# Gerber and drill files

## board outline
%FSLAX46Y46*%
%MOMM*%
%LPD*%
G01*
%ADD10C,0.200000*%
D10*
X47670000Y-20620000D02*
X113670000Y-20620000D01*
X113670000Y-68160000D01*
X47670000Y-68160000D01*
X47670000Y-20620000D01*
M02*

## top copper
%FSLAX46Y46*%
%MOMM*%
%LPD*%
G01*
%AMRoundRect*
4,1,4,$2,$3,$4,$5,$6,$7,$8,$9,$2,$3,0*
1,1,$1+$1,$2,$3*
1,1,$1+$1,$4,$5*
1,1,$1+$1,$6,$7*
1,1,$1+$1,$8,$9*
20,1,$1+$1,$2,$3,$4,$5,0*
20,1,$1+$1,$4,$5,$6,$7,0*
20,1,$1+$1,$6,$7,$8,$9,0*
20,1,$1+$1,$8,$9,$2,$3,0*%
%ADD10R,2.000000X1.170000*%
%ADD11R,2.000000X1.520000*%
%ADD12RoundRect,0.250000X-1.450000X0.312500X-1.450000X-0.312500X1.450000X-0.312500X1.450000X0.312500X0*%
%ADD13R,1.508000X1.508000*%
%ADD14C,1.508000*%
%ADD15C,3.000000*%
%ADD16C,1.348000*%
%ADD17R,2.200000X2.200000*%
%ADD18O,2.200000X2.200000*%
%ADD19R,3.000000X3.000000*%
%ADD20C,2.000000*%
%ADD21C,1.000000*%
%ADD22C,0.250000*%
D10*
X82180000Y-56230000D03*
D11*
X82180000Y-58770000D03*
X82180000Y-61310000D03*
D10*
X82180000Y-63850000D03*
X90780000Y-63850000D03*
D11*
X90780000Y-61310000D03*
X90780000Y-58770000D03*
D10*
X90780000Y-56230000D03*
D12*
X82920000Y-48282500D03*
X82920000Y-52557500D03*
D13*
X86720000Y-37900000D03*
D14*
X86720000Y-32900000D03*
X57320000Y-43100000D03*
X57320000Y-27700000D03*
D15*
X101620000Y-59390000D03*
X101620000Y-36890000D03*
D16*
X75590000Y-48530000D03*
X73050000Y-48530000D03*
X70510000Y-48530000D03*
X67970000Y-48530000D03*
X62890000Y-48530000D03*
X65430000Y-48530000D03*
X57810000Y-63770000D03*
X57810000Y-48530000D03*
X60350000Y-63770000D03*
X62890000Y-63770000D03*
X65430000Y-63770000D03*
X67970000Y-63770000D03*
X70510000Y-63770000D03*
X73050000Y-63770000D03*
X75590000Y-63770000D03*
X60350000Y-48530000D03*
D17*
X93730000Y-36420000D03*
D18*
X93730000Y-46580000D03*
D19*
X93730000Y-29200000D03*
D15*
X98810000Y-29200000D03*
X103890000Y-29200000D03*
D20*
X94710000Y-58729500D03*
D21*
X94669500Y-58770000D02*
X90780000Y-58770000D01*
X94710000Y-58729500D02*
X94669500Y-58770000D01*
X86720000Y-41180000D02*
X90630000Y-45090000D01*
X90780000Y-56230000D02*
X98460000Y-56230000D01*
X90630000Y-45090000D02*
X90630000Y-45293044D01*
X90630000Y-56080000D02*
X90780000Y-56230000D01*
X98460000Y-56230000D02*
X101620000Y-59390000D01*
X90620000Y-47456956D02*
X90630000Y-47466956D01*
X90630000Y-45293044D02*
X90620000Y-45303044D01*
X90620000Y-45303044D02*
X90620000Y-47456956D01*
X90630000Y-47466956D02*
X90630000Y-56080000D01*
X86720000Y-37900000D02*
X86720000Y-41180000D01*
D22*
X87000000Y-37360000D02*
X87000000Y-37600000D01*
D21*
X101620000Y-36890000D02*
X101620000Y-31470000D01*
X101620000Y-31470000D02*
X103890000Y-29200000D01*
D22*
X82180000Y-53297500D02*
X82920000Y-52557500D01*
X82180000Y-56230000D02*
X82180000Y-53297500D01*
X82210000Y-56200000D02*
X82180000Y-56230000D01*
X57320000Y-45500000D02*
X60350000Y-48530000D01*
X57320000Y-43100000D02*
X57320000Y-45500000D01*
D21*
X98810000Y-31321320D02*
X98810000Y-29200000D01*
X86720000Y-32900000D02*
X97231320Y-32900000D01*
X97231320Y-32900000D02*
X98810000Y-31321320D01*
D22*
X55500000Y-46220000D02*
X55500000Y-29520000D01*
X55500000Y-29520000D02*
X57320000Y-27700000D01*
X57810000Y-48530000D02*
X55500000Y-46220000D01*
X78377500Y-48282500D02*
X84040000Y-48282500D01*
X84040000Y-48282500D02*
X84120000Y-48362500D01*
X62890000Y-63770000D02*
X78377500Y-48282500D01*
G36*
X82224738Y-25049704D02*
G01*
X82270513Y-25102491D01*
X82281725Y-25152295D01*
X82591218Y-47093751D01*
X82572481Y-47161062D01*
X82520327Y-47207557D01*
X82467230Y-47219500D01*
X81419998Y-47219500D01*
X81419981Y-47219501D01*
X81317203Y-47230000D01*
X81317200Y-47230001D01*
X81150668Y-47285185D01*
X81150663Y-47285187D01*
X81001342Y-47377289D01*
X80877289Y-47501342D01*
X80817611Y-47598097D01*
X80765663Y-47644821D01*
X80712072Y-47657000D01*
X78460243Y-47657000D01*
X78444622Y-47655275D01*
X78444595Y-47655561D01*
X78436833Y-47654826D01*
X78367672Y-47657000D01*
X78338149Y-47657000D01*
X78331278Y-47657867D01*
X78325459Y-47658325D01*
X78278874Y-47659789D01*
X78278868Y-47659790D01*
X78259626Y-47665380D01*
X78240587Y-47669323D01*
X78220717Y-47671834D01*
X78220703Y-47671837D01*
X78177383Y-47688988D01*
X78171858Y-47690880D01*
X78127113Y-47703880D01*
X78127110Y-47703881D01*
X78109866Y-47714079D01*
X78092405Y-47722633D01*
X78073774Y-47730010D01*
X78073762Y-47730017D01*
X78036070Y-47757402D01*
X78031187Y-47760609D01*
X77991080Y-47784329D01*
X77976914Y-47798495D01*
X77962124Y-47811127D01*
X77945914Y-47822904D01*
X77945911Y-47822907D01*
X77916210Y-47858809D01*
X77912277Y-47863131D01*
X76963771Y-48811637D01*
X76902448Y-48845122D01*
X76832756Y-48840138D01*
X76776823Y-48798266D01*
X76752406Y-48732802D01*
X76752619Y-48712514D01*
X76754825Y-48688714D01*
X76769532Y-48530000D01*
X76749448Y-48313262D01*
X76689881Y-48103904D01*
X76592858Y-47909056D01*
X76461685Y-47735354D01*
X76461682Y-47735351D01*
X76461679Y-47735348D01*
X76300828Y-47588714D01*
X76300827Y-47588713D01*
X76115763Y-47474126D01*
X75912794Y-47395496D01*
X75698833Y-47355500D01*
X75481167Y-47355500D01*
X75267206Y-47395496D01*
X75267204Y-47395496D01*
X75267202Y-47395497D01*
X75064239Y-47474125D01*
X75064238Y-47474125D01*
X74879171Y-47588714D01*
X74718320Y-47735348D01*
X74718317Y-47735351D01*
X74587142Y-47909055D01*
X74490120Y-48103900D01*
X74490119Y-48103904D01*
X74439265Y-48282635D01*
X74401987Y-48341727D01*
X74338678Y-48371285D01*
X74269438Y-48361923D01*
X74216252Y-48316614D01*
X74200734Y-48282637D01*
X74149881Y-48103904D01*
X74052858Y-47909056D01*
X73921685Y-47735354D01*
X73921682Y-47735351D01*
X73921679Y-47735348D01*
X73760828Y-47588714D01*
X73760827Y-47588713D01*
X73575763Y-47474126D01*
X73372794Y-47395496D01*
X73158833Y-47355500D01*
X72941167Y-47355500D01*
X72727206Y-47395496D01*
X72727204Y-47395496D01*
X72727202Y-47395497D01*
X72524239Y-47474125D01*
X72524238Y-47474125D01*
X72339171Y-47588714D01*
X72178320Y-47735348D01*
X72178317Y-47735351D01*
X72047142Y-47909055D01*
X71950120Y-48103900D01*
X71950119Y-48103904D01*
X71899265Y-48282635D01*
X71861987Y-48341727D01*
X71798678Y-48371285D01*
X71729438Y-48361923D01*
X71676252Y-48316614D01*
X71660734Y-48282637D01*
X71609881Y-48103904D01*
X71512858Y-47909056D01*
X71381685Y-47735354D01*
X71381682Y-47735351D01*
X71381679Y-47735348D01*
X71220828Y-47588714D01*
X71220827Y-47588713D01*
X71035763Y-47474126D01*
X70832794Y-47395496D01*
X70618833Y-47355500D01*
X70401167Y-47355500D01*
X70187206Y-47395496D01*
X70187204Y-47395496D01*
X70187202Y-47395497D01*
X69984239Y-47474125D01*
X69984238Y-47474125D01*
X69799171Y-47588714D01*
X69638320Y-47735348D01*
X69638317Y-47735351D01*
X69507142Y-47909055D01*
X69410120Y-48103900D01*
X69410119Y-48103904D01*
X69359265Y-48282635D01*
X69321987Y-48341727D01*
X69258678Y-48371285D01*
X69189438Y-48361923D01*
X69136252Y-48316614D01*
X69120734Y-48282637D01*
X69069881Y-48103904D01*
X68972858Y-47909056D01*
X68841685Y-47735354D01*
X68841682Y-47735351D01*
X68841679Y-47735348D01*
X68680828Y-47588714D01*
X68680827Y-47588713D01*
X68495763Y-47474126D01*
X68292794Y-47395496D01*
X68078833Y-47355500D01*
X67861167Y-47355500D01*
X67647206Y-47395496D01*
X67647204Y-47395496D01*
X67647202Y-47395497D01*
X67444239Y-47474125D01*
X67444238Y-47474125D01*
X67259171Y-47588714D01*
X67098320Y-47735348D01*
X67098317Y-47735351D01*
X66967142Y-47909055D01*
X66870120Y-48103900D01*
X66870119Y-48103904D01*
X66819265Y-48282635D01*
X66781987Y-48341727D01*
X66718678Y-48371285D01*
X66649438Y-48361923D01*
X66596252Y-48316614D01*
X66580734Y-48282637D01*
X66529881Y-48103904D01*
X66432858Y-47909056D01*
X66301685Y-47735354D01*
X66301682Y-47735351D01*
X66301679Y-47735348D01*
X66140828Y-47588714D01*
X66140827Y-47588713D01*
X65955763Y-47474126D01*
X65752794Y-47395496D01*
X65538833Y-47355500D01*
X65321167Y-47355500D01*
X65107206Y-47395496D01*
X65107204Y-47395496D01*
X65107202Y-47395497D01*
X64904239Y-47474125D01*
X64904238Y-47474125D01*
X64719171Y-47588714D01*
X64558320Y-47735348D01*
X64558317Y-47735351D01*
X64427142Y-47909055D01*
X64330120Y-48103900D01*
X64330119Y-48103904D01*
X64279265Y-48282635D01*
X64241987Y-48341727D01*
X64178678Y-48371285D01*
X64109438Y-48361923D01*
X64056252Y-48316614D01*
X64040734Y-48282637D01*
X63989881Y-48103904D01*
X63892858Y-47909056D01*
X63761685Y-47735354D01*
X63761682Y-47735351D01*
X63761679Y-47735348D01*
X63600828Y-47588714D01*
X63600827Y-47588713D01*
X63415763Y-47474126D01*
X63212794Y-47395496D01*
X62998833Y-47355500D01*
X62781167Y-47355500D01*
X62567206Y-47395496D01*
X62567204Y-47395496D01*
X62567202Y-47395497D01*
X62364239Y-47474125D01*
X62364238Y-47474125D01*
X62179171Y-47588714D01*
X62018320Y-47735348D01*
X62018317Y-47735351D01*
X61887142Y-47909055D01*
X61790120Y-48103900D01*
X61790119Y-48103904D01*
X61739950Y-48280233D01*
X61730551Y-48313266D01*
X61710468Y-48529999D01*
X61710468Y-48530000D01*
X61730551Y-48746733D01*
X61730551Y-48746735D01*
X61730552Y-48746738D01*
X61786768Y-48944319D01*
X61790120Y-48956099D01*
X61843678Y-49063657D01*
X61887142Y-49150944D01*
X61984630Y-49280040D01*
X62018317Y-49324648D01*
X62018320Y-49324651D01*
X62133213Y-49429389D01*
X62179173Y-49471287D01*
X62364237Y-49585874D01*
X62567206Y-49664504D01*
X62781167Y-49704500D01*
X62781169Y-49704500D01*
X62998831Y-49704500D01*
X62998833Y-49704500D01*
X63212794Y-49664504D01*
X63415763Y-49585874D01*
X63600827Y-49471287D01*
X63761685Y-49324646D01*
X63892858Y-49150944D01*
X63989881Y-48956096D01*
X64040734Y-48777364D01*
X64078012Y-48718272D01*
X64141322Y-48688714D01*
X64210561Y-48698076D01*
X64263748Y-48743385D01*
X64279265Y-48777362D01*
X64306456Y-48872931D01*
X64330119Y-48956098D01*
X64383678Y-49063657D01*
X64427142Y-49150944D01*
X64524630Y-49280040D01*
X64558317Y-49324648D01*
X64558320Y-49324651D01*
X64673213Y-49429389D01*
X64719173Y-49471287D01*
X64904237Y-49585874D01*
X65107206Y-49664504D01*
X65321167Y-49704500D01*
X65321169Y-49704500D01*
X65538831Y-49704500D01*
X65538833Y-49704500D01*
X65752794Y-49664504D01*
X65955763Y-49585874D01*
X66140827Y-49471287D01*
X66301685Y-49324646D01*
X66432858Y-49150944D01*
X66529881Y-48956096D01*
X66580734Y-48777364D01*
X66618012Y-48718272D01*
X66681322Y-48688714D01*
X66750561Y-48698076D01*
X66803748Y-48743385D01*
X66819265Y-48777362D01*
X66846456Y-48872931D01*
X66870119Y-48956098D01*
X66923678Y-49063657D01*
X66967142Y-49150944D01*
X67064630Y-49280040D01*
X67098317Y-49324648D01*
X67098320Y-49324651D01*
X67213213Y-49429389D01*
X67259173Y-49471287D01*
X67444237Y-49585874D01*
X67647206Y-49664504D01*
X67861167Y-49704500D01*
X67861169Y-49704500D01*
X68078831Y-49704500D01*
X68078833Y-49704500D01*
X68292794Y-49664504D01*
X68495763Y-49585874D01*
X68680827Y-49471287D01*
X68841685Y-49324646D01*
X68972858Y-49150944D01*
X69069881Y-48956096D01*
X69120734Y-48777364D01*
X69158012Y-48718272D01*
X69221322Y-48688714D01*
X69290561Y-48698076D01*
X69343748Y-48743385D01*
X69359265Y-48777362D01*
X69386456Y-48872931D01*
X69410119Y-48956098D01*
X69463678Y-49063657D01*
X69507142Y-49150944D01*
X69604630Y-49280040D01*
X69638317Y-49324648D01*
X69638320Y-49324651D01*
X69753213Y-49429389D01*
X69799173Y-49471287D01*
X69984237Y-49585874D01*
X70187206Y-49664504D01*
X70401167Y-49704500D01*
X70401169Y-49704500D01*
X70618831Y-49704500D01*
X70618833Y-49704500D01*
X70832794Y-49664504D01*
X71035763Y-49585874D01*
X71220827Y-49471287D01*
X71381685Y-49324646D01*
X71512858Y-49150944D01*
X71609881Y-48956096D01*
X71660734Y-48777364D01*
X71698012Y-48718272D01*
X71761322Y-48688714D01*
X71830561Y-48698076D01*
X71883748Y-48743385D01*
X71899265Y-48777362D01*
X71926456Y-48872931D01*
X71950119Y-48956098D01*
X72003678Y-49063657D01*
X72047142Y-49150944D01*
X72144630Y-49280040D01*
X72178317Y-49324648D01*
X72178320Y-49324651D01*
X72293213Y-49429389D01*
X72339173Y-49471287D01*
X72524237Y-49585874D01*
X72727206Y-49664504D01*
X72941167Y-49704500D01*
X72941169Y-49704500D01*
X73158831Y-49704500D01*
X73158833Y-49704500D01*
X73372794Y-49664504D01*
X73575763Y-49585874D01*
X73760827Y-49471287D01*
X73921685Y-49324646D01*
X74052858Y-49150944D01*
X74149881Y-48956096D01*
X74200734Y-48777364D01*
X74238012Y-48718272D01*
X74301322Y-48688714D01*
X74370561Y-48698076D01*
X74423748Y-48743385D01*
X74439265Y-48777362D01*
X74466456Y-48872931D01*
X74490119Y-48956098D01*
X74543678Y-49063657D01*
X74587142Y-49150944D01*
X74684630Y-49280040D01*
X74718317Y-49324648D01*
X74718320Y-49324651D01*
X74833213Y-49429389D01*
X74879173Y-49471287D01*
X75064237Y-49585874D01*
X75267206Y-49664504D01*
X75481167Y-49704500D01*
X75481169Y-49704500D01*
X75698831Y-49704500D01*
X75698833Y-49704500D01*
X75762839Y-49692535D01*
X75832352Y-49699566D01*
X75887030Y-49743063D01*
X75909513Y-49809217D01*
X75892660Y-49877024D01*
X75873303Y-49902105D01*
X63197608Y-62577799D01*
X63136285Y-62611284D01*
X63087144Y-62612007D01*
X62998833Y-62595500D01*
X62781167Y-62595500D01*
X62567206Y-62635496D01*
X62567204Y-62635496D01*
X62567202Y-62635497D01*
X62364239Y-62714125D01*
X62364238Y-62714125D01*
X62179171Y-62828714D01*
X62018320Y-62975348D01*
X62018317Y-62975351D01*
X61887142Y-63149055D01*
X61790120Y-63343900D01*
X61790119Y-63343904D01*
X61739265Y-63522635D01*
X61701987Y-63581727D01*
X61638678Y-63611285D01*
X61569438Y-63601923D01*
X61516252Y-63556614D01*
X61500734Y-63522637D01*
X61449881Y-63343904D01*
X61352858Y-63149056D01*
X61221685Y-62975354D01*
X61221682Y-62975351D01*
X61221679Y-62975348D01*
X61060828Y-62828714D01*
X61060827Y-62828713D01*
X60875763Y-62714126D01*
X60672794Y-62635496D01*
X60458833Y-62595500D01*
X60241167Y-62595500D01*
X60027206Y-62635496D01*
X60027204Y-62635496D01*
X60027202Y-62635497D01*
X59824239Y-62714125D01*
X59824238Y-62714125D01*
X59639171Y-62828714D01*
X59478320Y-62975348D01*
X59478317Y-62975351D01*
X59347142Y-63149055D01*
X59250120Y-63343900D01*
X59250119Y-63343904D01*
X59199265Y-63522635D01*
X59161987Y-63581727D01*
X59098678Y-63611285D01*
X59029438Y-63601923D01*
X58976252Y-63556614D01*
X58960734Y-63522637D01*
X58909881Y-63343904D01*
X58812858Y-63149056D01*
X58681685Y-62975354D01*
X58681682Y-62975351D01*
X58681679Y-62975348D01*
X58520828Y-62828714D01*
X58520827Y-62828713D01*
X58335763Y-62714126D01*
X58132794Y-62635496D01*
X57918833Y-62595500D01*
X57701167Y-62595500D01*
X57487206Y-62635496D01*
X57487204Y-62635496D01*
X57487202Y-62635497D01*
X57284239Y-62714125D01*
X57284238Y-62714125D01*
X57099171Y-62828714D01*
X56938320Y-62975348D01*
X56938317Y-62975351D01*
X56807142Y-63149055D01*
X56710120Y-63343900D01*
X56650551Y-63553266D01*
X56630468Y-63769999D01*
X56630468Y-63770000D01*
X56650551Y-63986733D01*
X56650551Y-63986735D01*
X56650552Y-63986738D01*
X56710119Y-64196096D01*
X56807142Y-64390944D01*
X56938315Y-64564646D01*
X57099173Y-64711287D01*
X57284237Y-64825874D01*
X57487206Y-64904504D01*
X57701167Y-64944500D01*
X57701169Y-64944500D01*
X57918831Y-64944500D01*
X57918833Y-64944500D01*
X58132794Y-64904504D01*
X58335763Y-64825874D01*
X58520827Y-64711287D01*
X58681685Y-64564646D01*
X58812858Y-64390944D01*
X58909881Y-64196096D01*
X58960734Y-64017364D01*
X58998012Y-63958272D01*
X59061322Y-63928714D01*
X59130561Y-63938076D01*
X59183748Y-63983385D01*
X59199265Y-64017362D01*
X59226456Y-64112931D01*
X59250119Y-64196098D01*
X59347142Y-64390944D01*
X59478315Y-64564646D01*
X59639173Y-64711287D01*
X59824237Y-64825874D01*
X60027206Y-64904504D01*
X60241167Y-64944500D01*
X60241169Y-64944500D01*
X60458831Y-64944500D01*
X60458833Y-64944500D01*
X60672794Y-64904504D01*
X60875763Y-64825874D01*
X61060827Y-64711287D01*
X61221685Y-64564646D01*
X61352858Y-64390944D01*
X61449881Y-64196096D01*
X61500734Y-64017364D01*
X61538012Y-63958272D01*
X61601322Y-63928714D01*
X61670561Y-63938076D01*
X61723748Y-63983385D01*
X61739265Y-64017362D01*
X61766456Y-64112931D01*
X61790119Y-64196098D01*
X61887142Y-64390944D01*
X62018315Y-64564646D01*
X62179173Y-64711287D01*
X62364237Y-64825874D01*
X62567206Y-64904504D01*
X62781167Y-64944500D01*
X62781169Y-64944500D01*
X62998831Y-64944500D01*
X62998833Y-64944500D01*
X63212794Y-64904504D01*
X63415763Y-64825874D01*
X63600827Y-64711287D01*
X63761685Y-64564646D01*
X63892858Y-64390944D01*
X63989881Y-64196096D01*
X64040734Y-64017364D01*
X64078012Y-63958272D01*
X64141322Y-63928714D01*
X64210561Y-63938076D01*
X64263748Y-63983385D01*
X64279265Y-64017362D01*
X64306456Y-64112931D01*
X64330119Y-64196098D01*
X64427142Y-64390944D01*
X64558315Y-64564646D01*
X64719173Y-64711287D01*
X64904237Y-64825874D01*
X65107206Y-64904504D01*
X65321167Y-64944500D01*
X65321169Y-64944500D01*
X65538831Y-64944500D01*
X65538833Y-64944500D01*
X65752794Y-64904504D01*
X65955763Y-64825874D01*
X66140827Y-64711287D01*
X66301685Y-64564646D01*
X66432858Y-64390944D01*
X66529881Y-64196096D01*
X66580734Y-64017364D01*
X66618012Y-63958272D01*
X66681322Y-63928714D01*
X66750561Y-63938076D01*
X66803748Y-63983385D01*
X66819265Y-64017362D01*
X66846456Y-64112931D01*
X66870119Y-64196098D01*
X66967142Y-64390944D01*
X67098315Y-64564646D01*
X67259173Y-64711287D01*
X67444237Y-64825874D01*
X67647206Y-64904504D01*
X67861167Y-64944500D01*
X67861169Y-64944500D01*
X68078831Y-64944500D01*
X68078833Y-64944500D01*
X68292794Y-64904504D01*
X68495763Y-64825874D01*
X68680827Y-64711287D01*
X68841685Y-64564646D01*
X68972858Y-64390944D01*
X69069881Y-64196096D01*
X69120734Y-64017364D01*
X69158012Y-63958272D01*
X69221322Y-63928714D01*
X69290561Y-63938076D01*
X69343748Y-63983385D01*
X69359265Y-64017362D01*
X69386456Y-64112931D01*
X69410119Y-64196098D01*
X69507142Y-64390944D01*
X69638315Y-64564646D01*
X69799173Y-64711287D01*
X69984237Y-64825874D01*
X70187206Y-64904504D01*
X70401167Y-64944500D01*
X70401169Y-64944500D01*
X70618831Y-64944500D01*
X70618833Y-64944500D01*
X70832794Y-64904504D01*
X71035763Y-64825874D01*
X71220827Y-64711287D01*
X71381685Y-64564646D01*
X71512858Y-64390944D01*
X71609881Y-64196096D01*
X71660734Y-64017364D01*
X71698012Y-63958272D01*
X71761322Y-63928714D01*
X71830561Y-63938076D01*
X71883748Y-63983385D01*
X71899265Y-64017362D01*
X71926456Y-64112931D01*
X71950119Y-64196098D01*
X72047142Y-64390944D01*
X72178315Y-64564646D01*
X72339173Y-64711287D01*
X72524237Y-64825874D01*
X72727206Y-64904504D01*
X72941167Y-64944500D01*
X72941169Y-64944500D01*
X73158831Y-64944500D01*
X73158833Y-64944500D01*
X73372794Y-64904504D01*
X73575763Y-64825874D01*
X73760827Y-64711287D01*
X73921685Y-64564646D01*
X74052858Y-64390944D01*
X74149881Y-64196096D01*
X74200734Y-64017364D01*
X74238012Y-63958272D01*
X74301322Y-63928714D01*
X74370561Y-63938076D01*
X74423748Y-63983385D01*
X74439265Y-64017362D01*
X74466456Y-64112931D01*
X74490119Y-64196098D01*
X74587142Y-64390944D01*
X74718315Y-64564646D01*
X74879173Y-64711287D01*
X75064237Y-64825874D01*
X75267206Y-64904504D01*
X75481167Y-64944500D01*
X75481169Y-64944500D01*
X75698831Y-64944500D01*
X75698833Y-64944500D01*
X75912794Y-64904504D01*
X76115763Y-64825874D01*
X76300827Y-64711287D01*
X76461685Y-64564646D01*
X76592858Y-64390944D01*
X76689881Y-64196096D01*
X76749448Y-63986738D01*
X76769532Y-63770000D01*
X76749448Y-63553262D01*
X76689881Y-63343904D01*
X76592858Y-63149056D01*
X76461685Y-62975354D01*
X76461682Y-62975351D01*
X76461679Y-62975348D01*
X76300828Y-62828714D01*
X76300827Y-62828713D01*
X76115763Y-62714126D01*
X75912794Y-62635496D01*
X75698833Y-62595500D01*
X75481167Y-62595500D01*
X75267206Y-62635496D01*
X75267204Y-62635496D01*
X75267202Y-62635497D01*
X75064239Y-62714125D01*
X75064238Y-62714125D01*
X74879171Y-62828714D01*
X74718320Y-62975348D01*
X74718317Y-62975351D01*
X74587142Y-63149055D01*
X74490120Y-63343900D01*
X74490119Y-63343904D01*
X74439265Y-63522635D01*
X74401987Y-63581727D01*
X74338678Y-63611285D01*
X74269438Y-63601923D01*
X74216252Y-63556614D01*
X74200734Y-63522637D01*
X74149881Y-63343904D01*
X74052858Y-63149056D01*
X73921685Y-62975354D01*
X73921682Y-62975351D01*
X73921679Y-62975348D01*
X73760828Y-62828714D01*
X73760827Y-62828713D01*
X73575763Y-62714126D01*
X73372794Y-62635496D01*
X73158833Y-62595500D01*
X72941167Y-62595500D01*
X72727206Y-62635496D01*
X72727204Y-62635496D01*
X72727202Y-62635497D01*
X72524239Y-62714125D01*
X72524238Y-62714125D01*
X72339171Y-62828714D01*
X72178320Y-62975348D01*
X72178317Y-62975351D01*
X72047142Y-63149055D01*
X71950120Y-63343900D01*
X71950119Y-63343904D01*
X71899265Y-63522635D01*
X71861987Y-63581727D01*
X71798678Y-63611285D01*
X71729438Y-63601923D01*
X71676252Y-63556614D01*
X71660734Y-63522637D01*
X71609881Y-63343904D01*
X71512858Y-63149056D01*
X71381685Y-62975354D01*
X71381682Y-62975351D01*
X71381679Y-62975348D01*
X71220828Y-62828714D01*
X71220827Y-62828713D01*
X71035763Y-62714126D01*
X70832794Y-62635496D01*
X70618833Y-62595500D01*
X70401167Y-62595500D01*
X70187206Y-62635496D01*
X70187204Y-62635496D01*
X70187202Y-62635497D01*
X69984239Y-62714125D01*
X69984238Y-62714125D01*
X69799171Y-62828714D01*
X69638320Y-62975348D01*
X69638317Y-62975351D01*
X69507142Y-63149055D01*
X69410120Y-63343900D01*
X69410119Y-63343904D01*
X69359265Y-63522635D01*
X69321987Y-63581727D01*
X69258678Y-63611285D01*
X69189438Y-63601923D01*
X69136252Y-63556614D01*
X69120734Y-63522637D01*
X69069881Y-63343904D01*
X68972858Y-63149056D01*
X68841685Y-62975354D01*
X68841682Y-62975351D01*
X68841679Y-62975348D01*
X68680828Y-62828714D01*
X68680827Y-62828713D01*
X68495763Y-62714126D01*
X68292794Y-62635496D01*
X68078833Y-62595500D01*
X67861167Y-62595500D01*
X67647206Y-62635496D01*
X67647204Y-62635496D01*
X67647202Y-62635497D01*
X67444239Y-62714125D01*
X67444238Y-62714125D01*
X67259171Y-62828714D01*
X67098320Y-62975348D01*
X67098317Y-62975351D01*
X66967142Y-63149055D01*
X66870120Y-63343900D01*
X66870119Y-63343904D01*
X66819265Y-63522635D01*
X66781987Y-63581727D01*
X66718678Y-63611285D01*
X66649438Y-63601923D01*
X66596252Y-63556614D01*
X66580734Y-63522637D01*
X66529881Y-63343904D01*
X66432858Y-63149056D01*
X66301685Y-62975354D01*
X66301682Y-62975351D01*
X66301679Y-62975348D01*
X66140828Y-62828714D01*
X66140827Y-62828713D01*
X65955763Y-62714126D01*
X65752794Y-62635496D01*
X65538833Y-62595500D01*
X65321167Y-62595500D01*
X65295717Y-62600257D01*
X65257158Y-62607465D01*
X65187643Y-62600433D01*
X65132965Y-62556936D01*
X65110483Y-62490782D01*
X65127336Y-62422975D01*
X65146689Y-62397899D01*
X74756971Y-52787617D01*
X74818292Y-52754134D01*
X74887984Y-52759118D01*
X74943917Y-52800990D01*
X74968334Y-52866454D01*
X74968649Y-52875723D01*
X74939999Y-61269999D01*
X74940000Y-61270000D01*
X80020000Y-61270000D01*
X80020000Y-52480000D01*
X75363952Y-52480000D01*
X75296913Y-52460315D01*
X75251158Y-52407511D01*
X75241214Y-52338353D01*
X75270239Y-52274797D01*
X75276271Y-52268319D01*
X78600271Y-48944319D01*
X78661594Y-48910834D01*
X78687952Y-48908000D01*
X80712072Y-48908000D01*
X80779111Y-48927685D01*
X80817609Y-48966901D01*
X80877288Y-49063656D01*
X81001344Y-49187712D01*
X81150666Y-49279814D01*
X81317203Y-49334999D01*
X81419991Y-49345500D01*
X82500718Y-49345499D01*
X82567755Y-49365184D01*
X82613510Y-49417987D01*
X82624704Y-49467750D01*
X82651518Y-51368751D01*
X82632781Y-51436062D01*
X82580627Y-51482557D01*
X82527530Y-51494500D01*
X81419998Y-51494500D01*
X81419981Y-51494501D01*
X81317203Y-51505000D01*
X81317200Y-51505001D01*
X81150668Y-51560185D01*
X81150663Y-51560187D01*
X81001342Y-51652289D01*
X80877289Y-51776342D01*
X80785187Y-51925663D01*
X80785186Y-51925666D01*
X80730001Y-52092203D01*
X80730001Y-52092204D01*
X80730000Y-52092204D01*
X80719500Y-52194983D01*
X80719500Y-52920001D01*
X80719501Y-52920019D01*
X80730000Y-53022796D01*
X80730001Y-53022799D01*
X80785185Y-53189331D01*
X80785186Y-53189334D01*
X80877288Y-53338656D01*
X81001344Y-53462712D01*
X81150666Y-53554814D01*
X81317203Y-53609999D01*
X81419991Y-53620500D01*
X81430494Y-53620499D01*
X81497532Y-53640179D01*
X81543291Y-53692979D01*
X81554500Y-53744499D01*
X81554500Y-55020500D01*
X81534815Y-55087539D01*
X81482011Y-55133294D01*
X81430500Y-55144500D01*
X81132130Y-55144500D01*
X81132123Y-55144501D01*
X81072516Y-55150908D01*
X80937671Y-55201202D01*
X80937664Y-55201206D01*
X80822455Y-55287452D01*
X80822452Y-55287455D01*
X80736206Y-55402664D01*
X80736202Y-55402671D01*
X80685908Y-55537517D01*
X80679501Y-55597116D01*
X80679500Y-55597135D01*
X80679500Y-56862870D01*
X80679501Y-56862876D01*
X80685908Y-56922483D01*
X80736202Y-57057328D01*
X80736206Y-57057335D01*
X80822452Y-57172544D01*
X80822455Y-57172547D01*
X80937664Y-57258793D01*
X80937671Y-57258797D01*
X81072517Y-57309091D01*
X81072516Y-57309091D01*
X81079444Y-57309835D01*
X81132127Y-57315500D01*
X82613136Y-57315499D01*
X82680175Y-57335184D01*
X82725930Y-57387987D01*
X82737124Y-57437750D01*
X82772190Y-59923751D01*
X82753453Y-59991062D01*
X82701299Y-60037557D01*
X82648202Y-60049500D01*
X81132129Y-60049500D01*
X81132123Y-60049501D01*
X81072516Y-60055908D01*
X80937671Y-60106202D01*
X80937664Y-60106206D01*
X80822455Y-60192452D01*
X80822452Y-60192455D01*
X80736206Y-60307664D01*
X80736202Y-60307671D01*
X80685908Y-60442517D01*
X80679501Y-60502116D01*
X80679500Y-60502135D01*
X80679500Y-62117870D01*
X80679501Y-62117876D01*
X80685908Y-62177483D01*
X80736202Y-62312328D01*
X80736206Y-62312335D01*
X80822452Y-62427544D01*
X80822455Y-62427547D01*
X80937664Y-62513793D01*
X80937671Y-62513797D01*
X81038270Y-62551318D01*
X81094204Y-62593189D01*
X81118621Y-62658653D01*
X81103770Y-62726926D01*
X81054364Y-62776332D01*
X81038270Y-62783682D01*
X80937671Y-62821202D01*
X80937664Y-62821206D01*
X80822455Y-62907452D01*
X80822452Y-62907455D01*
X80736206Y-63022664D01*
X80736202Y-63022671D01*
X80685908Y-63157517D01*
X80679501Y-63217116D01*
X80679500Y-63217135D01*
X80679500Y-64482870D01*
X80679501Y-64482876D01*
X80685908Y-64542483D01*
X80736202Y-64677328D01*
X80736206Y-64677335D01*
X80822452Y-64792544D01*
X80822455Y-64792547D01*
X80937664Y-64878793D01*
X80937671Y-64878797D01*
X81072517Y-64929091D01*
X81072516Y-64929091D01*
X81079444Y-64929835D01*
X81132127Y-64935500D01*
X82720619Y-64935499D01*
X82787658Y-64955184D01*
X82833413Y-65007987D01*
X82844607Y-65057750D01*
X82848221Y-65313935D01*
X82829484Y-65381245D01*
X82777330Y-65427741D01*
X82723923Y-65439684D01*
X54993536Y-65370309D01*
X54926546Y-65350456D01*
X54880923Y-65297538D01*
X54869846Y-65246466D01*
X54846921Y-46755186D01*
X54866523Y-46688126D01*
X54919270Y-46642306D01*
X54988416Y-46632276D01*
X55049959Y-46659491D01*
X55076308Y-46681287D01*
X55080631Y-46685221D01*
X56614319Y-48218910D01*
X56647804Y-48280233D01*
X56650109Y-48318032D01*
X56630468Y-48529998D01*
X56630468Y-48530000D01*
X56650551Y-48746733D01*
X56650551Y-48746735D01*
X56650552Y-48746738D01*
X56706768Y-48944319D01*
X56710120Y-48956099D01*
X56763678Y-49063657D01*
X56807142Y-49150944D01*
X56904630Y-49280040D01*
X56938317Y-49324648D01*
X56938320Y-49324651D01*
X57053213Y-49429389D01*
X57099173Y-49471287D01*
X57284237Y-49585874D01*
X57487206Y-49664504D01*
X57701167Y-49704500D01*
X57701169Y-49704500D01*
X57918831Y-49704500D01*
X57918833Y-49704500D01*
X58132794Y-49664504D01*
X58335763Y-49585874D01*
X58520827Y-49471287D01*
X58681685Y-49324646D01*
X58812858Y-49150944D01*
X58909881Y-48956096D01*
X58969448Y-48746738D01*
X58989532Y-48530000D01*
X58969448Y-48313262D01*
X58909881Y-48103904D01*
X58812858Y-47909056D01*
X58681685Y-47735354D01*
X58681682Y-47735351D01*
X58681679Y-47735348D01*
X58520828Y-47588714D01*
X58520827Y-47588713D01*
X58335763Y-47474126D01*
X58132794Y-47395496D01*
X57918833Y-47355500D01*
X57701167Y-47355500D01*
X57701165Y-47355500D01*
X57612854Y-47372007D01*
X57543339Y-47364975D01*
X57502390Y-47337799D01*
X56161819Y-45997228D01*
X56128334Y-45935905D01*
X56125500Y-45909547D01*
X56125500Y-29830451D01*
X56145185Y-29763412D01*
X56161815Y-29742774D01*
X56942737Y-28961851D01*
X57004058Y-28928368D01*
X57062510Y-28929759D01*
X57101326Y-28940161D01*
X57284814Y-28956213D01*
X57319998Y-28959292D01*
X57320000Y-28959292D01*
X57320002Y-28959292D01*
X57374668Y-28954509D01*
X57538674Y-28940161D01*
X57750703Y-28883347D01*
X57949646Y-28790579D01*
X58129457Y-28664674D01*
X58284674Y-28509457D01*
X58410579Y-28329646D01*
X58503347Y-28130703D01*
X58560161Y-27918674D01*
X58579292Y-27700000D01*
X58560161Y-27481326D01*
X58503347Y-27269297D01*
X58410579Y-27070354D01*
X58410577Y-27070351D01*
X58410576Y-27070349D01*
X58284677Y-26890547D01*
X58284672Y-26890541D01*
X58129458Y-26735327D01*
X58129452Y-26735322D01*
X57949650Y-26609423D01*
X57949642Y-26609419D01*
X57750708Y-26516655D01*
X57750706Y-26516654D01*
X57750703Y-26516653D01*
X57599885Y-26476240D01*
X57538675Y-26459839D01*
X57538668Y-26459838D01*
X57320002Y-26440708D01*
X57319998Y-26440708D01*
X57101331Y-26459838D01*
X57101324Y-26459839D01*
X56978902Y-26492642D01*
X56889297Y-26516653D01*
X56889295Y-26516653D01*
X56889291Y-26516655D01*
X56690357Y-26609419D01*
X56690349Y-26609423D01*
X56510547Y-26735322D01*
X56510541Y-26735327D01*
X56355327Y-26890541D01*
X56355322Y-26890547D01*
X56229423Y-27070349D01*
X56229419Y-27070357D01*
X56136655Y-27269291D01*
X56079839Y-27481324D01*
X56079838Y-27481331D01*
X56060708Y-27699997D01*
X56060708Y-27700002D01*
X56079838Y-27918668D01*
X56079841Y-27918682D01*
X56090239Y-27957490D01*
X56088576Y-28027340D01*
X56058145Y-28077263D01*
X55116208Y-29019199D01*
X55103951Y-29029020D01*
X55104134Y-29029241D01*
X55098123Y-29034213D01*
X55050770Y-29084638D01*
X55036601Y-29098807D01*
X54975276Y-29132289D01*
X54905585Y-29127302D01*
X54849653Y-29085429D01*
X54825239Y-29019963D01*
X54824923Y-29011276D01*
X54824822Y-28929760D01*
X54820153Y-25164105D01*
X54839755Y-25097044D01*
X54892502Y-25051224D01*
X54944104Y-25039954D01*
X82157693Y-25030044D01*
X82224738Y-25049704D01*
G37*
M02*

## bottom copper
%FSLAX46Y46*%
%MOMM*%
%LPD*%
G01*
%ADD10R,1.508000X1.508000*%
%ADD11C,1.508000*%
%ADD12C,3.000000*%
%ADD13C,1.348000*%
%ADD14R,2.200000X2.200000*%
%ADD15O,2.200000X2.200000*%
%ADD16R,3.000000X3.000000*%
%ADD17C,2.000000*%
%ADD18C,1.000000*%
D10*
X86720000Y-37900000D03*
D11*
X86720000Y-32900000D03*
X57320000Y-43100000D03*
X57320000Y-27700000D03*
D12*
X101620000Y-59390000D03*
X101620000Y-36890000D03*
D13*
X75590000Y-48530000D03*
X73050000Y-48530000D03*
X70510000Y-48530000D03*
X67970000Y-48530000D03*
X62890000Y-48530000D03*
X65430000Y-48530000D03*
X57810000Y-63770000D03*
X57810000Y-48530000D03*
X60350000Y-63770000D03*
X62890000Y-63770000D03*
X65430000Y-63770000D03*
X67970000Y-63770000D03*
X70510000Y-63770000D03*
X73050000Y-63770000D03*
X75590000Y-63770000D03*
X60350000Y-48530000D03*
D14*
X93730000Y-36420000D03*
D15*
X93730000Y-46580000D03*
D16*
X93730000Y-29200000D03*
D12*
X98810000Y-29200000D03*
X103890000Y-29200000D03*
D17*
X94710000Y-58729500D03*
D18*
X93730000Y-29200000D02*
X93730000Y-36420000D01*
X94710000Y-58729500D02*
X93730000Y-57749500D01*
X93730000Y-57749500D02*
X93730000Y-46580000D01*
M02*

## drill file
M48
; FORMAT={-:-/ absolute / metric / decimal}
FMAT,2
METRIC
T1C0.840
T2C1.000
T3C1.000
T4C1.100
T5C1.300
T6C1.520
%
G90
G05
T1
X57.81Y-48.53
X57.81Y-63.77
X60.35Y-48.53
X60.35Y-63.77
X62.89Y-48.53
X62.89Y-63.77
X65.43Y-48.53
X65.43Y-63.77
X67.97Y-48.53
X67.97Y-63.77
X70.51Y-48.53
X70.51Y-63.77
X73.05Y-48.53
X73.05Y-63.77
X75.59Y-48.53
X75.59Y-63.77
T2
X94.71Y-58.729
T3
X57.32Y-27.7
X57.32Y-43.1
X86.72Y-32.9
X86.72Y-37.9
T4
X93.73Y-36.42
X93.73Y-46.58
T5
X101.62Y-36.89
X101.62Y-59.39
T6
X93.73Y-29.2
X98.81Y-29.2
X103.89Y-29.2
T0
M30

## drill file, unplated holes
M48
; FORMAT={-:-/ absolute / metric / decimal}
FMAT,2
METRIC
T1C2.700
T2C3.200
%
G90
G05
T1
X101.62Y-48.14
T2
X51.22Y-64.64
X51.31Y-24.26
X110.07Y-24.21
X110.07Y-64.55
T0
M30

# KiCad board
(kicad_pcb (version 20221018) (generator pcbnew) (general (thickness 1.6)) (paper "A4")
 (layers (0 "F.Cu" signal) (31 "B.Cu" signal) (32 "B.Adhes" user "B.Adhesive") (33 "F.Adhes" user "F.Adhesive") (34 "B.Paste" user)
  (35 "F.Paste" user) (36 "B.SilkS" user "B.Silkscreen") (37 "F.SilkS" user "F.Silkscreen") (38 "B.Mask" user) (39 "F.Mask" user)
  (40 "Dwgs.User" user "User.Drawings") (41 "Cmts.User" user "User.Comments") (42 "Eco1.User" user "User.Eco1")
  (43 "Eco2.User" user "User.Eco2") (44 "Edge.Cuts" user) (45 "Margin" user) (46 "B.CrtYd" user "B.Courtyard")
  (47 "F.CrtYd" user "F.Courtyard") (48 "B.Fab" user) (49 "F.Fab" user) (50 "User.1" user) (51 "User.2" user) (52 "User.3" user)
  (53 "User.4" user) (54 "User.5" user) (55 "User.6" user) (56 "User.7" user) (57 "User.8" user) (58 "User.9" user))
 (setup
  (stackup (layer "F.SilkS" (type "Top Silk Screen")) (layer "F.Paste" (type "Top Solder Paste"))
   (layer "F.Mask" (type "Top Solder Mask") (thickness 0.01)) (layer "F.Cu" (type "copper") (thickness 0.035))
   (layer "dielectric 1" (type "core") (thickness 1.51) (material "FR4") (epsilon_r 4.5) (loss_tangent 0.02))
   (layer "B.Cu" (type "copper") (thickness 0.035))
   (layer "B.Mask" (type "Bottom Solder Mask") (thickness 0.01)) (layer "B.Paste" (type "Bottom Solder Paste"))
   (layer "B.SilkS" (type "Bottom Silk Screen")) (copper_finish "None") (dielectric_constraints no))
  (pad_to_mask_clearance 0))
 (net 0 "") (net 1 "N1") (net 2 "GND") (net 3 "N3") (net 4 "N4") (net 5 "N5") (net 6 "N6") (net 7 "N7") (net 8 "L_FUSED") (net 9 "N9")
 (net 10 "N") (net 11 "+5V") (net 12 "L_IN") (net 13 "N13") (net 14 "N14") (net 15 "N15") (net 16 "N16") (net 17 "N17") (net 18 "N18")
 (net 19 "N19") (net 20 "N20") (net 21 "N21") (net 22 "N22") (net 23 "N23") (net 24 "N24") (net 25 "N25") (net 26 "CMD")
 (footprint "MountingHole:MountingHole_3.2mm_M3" (layer "F.Cu") (at 110.07 24.21)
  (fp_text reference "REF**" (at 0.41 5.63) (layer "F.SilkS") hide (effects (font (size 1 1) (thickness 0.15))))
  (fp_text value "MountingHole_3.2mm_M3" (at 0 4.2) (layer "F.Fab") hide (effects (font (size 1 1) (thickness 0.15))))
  (pad "" np_thru_hole circle (at 0 0) (size 3.2 3.2) (drill 3.2) (layers "F&B.Cu" "*.Mask")))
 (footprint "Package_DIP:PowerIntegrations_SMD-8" (layer "F.Cu") (at 86.48 60.04)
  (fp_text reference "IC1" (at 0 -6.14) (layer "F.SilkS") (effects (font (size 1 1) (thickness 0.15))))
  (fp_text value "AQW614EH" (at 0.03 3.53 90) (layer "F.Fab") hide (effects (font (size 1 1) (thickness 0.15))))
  (pad "1" smd rect (at -4.3 -3.81) (size 2 1.17) (layers "F.Cu" "F.Paste" "F.Mask") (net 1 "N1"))
  (pad "2" smd rect (at -4.3 -1.27) (size 2 1.52) (layers "F.Cu" "F.Paste" "F.Mask") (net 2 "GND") (zone_connect 2))
  (pad "3" smd rect (at -4.3 1.27) (size 2 1.52) (layers "F.Cu" "F.Paste" "F.Mask") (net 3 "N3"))
  (pad "4" smd rect (at -4.3 3.81) (size 2 1.17) (layers "F.Cu" "F.Paste" "F.Mask") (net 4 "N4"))
  (pad "5" smd rect (at 4.3 3.81) (size 2 1.17) (layers "F.Cu" "F.Paste" "F.Mask") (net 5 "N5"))
  (pad "6" smd rect (at 4.3 1.27) (size 2 1.52) (layers "F.Cu" "F.Paste" "F.Mask") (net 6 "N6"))
  (pad "7" smd rect (at 4.3 -1.27) (size 2 1.52) (layers "F.Cu" "F.Paste" "F.Mask") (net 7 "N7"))
  (pad "8" smd rect (at 4.3 -3.81) (size 2 1.17) (layers "F.Cu" "F.Paste" "F.Mask") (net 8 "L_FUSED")))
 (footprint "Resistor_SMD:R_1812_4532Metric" (layer "F.Cu") (at 82.92 50.42 -90)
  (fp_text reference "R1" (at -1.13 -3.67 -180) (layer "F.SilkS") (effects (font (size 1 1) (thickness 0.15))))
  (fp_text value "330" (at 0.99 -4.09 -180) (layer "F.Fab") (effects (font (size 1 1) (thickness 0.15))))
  (pad "1" smd roundrect (at -2.1375 0 270) (size 1.125 3.4) (layers "F.Cu" "F.Paste" "F.Mask") (roundrect_rratio 0.2222222222) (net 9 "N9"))
  (pad "2" smd roundrect (at 2.1375 0 270) (size 1.125 3.4) (layers "F.Cu" "F.Paste" "F.Mask") (roundrect_rratio 0.2222222222) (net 1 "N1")))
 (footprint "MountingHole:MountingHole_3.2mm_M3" (layer "F.Cu") (at 110.07 64.55)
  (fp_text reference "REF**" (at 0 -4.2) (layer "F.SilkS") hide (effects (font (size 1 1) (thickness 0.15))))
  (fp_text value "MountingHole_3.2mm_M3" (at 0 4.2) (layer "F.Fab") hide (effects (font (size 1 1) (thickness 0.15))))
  (pad "" np_thru_hole circle (at 0 0) (size 3.2 3.2) (drill 3.2) (layers "F&B.Cu" "*.Mask")))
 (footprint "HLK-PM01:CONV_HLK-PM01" (layer "F.Cu") (at 72.02 35.4 180)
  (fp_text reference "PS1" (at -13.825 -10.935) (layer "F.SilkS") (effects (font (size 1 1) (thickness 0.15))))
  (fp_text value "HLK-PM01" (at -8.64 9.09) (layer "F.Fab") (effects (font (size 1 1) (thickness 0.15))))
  (pad "1" thru_hole rect (at -14.7 -2.5 180) (size 1.508 1.508) (drill 1) (layers "*.Cu" "*.Mask") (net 8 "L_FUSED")
   (solder_mask_margin 0.102))
  (pad "2" thru_hole circle (at -14.7 2.5 180) (size 1.508 1.508) (drill 1) (layers "*.Cu" "*.Mask") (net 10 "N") (solder_mask_margin 0.102))
  (pad "3" thru_hole circle (at 14.7 -7.7 180) (size 1.508 1.508) (drill 1) (layers "*.Cu" "*.Mask") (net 2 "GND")
   (solder_mask_margin 0.102) (zone_connect 2))
  (pad "4" thru_hole circle (at 14.7 7.7 180) (size 1.508 1.508) (drill 1) (layers "*.Cu" "*.Mask") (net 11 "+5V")
   (solder_mask_margin 0.102)))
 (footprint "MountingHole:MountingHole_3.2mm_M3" (layer "F.Cu") (at 51.22 64.64)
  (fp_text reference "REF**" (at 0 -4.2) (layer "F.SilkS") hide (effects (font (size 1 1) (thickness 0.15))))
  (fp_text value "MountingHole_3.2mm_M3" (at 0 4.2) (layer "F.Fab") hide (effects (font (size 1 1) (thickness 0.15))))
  (pad "" np_thru_hole circle (at 0 0) (size 3.2 3.2) (drill 3.2) (layers "F&B.Cu" "*.Mask")))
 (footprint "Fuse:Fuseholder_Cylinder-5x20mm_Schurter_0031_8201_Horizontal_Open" (layer "F.Cu") (at 101.62 59.39 90)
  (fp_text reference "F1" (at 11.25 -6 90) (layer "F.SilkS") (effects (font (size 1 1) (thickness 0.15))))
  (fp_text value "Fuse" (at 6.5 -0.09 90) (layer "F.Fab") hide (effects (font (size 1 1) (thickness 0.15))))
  (pad "" np_thru_hole circle (at 11.25 0 90) (size 2.7 2.7) (drill 2.7) (layers "*.Cu" "*.Mask"))
  (pad "1" thru_hole circle (at 0 0 90) (size 3 3) (drill 1.3) (layers "*.Cu" "*.Mask") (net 8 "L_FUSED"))
  (pad "2" thru_hole circle (at 22.5 0 90) (size 3 3) (drill 1.3) (layers "*.Cu" "*.Mask") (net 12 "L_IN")))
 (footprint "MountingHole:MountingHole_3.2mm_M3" (layer "F.Cu") (at 51.31 24.26)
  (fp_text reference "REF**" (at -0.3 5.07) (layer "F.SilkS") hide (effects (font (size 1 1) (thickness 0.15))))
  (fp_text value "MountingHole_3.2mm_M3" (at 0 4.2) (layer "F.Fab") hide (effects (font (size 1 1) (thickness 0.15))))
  (pad "" np_thru_hole circle (at 0 0) (size 3.2 3.2) (drill 3.2) (layers "*.Cu" "*.Mask")))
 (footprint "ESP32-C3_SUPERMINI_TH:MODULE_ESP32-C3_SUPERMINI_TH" (layer "F.Cu") (at 67.71 56.15 90)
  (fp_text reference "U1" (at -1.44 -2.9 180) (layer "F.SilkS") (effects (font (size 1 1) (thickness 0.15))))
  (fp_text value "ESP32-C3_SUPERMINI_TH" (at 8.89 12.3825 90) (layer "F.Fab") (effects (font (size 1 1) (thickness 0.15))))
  (pad "0" thru_hole circle (at 7.62 7.88 90) (size 1.348 1.348) (drill 0.84) (layers "*.Cu" "*.Mask") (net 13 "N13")
   (solder_mask_margin 0.102))
  (pad "1" thru_hole circle (at 7.62 5.34 90) (size 1.348 1.348) (drill 0.84) (layers "*.Cu" "*.Mask") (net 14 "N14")
   (solder_mask_margin 0.102))
  (pad "2" thru_hole circle (at 7.62 2.8 90) (size 1.348 1.348) (drill 0.84) (layers "*.Cu" "*.Mask") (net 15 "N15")
   (solder_mask_margin 0.102))
  (pad "3" thru_hole circle (at 7.62 0.26 90) (size 1.348 1.348) (drill 0.84) (layers "*.Cu" "*.Mask") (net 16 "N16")
   (solder_mask_margin 0.102))
  (pad "3.3" thru_hole circle (at 7.62 -4.82 90) (size 1.348 1.348) (drill 0.84) (layers "*.Cu" "*.Mask") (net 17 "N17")
   (solder_mask_margin 0.102))
  (pad "4" thru_hole circle (at 7.62 -2.28 90) (size 1.348 1.348) (drill 0.84) (layers "*.Cu" "*.Mask") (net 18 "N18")
   (solder_mask_margin 0.102))
  (pad "5" thru_hole circle (at -7.62 -9.9 90) (size 1.348 1.348) (drill 0.84) (layers "*.Cu" "*.Mask") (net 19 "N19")
   (solder_mask_margin 0.102))
  (pad "5V" thru_hole circle (at 7.62 -9.9 90) (size 1.348 1.348) (drill 0.84) (layers "*.Cu" "*.Mask") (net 11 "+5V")
   (solder_mask_margin 0.102))
  (pad "6" thru_hole circle (at -7.62 -7.36 90) (size 1.348 1.348) (drill 0.84) (layers "*.Cu" "*.Mask") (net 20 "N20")
   (solder_mask_margin 0.102))
  (pad "7" thru_hole circle (at -7.62 -4.82 90) (size 1.348 1.348) (drill 0.84) (layers "*.Cu" "*.Mask") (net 9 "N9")
   (solder_mask_margin 0.102))
  (pad "8" thru_hole circle (at -7.62 -2.28 90) (size 1.348 1.348) (drill 0.84) (layers "*.Cu" "*.Mask") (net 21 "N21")
   (solder_mask_margin 0.102))
  (pad "9" thru_hole circle (at -7.62 0.26 90) (size 1.348 1.348) (drill 0.84) (layers "*.Cu" "*.Mask") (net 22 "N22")
   (solder_mask_margin 0.102))
  (pad "10" thru_hole circle (at -7.62 2.8 90) (size 1.348 1.348) (drill 0.84) (layers "*.Cu" "*.Mask") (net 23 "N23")
   (solder_mask_margin 0.102))
  (pad "20" thru_hole circle (at -7.62 5.34 90) (size 1.348 1.348) (drill 0.84) (layers "*.Cu" "*.Mask") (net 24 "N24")
   (solder_mask_margin 0.102))
  (pad "21" thru_hole circle (at -7.62 7.88 90) (size 1.348 1.348) (drill 0.84) (layers "*.Cu" "*.Mask") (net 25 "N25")
   (solder_mask_margin 0.102))
  (pad "G" thru_hole circle (at 7.62 -7.36 90) (size 1.348 1.348) (drill 0.84) (layers "*.Cu" "*.Mask") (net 2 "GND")
   (solder_mask_margin 0.102) (zone_connect 2)))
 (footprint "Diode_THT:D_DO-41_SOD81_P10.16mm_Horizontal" (layer "F.Cu") (at 93.73 36.42 -90)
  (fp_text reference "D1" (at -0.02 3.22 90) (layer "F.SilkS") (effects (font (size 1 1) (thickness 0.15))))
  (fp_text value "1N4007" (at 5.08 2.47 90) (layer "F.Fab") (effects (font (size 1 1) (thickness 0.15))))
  (pad "1" thru_hole rect (at 0 0 270) (size 2.2 2.2) (drill 1.1) (layers "*.Cu" "*.Mask") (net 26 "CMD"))
  (pad "2" thru_hole oval (at 10.16 0 270) (size 2.2 2.2) (drill 1.1) (layers "*.Cu" "*.Mask") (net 7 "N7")))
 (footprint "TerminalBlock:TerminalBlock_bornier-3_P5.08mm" (layer "F.Cu") (at 93.73 29.2)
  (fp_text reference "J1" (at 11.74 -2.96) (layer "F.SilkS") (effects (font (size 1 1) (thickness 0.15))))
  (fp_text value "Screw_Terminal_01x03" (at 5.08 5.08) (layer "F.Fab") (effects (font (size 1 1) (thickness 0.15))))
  (pad "1" thru_hole rect (at 0 0) (size 3 3) (drill 1.52) (layers "*.Cu" "*.Mask") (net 26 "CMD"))
  (pad "2" thru_hole circle (at 5.08 0) (size 3 3) (drill 1.52) (layers "*.Cu" "*.Mask") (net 10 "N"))
  (pad "3" thru_hole circle (at 10.16 0) (size 3 3) (drill 1.52) (layers "*.Cu" "*.Mask") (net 12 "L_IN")))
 (gr_rect (start 47.67 20.62) (end 113.67 68.16) (stroke (width 0.2) (type default)) (fill none) (layer "Edge.Cuts"))
 (segment (start 93.73 29.2) (end 93.73 36.42) (width 1) (layer "B.Cu") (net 26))
 (segment (start 94.6695 58.77) (end 90.78 58.77) (width 1) (layer "F.Cu") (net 7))
 (segment (start 94.71 58.7295) (end 94.6695 58.77) (width 1) (layer "F.Cu") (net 7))
 (via (at 94.71 58.7295) (size 2) (drill 1) (layers "F.Cu" "B.Cu") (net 7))
 (segment (start 94.71 58.7295) (end 93.73 57.7495) (width 1) (layer "B.Cu") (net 7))
 (segment (start 93.73 57.7495) (end 93.73 46.58) (width 1) (layer "B.Cu") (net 7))
 (segment (start 86.72 41.18) (end 90.63 45.09) (width 1) (layer "F.Cu") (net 8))
 (segment (start 90.78 56.23) (end 98.46 56.23) (width 1) (layer "F.Cu") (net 8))
 (segment (start 90.63 45.09) (end 90.63 45.293044) (width 1) (layer "F.Cu") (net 8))
 (segment (start 90.63 56.08) (end 90.78 56.23) (width 1) (layer "F.Cu") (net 8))
 (segment (start 98.46 56.23) (end 101.62 59.39) (width 1) (layer "F.Cu") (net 8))
 (segment (start 90.62 47.456956) (end 90.63 47.466956) (width 1) (layer "F.Cu") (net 8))
 (segment (start 90.63 45.293044) (end 90.62 45.303044) (width 1) (layer "F.Cu") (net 8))
 (segment (start 90.62 45.303044) (end 90.62 47.456956) (width 1) (layer "F.Cu") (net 8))
 (segment (start 90.63 47.466956) (end 90.63 56.08) (width 1) (layer "F.Cu") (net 8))
 (segment (start 86.72 37.9) (end 86.72 41.18) (width 1) (layer "F.Cu") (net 8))
 (segment (start 87 37.36) (end 87 37.6) (width 0.25) (layer "F.Cu") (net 8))
 (segment (start 101.62 36.89) (end 101.62 31.47) (width 1) (layer "F.Cu") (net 12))
 (segment (start 101.62 31.47) (end 103.89 29.2) (width 1) (layer "F.Cu") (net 12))
 (segment (start 82.18 53.2975) (end 82.92 52.5575) (width 0.25) (layer "F.Cu") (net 1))
 (segment (start 82.18 56.23) (end 82.18 53.2975) (width 0.25) (layer "F.Cu") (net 1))
 (segment (start 82.21 56.2) (end 82.18 56.23) (width 0.25) (layer "F.Cu") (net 1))
 (segment (start 57.32 45.5) (end 60.35 48.53) (width 0.25) (layer "F.Cu") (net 2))
 (segment (start 57.32 43.1) (end 57.32 45.5) (width 0.25) (layer "F.Cu") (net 2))
 (segment (start 98.81 31.32132) (end 98.81 29.2) (width 1) (layer "F.Cu") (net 10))
 (segment (start 86.72 32.9) (end 97.23132 32.9) (width 1) (layer "F.Cu") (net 10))
 (segment (start 97.23132 32.9) (end 98.81 31.32132) (width 1) (layer "F.Cu") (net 10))
 (segment (start 55.5 46.22) (end 55.5 29.52) (width 0.25) (layer "F.Cu") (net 11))
 (segment (start 55.5 29.52) (end 57.32 27.7) (width 0.25) (layer "F.Cu") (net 11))
 (segment (start 57.81 48.53) (end 55.5 46.22) (width 0.25) (layer "F.Cu") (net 11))
 (segment (start 78.3775 48.2825) (end 84.04 48.2825) (width 0.25) (layer "F.Cu") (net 9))
 (segment (start 84.04 48.2825) (end 84.12 48.3625) (width 0.25) (layer "F.Cu") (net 9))
 (segment (start 62.89 63.77) (end 78.3775 48.2825) (width 0.25) (layer "F.Cu") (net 9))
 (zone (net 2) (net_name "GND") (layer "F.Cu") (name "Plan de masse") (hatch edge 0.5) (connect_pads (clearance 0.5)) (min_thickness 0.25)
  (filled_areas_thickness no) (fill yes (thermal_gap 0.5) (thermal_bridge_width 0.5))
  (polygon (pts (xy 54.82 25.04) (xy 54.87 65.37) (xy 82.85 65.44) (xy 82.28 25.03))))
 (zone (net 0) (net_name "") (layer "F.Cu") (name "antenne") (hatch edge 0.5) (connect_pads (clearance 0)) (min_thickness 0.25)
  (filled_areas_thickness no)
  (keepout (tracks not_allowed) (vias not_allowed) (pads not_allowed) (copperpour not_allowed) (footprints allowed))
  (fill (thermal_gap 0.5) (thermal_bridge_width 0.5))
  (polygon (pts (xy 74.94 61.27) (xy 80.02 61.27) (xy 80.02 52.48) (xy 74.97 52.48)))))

